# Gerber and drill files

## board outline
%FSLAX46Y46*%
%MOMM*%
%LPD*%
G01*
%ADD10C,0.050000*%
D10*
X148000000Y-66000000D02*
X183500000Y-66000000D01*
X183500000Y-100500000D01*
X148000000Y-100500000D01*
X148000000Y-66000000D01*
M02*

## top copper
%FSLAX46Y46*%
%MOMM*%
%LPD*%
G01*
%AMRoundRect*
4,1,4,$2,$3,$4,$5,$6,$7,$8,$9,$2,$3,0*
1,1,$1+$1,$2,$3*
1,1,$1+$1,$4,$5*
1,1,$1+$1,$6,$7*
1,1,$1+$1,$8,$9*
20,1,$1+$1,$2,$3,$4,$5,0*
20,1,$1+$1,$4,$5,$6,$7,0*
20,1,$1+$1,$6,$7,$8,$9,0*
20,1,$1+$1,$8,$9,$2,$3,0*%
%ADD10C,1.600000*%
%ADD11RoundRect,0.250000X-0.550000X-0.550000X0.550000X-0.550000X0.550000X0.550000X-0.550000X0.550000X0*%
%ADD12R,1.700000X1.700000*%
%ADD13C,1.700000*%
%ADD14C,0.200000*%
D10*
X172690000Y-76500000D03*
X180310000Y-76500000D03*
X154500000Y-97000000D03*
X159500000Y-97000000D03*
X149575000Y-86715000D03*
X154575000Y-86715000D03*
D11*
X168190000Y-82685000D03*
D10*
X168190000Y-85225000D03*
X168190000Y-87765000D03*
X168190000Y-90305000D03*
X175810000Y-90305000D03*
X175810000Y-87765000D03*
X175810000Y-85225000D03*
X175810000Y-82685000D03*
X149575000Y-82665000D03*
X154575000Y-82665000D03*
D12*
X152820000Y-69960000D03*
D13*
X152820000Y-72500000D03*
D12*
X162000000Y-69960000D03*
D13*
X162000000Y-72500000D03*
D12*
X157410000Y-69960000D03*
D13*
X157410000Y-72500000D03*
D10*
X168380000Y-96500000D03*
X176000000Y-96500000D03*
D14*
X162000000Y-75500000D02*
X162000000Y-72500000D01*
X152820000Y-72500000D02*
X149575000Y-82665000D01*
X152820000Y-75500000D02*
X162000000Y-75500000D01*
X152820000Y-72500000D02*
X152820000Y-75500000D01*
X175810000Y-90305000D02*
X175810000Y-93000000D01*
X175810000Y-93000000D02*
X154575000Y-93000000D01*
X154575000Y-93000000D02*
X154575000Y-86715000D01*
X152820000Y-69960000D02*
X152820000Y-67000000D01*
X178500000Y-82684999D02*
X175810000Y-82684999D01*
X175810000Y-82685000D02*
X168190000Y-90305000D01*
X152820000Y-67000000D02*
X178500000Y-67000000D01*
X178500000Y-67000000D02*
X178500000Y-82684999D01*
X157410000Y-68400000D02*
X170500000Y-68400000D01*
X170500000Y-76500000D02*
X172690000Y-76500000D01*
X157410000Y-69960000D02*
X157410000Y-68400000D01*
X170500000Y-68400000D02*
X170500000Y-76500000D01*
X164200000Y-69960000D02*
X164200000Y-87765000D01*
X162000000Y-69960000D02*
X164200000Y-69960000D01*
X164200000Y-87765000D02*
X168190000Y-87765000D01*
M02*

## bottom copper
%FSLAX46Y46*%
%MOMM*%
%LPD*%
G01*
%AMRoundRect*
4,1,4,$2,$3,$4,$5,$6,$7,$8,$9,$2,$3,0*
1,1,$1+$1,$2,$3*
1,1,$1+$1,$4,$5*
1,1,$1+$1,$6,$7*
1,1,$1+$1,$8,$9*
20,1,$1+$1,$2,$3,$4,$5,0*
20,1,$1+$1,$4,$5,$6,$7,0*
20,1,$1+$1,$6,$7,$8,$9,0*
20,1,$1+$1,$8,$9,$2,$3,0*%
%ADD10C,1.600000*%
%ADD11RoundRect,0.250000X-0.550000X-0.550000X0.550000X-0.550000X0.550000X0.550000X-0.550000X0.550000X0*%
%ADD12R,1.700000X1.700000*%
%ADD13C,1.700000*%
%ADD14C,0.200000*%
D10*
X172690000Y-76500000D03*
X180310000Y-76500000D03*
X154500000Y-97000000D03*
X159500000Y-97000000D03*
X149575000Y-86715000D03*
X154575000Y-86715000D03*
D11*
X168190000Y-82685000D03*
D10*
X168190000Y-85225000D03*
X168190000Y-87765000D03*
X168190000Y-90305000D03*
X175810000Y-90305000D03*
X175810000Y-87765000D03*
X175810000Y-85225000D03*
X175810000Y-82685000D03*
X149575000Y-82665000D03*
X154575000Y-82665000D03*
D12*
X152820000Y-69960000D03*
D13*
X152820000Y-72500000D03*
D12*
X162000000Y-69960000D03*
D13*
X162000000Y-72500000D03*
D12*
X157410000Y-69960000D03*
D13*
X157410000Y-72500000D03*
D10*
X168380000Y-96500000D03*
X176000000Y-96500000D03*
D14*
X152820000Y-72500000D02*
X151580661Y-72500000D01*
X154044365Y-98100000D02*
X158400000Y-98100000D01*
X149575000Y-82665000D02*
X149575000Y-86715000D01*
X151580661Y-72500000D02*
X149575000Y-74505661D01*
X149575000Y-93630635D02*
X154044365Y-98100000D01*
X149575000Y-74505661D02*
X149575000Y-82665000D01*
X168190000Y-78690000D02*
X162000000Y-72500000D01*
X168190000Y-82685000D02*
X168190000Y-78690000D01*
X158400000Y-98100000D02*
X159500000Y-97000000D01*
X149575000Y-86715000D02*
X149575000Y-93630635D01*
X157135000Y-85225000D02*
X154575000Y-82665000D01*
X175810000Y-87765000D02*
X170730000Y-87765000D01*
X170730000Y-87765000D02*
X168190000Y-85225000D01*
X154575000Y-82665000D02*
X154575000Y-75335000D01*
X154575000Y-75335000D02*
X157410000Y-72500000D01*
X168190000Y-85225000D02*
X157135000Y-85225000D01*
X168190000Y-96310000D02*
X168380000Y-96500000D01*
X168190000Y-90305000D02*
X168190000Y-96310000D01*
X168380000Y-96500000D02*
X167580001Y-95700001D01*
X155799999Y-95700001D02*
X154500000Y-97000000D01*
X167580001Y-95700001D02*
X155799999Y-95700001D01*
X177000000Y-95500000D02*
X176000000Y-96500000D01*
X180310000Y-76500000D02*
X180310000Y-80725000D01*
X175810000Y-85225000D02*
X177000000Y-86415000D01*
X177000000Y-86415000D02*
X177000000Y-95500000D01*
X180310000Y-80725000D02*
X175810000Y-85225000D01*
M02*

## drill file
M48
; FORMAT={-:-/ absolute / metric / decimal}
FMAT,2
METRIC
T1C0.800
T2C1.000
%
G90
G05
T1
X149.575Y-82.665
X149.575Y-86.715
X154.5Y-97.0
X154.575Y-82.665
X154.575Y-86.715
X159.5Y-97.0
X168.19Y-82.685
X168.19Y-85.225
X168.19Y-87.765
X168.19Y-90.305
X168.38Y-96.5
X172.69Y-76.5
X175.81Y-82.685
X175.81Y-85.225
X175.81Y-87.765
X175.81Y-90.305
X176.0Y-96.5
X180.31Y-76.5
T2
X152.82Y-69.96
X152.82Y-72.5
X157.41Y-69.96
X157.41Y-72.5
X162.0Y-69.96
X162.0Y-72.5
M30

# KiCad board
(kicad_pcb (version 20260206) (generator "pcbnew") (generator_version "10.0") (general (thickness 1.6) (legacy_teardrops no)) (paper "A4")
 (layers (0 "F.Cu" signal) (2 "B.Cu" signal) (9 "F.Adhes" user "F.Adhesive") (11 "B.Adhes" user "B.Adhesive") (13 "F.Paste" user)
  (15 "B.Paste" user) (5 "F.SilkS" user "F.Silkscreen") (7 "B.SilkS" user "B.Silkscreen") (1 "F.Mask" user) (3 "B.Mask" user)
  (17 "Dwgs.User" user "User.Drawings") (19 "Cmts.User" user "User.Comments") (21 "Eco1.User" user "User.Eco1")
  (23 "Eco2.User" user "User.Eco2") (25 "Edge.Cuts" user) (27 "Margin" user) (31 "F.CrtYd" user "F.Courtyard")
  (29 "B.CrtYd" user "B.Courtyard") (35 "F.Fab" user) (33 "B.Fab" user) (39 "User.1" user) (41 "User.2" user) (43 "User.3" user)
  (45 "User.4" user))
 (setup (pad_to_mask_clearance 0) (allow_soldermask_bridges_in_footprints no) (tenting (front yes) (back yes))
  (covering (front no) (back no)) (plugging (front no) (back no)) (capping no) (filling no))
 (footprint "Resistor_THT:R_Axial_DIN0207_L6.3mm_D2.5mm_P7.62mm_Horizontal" (layer "F.Cu") (at 172.69 76.5)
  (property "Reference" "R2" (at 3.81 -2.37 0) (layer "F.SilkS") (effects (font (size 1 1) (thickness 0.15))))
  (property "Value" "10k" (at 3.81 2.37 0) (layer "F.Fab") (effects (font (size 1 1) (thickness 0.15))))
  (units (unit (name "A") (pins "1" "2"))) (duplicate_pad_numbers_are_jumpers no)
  (pad "1" thru_hole circle (at 0 0) (size 1.6 1.6) (drill 0.8) (layers "*.Cu" "*.Mask") (remove_unused_layers no) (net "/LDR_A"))
  (pad "2" thru_hole circle (at 7.62 0) (size 1.6 1.6) (drill 0.8) (layers "*.Cu" "*.Mask") (remove_unused_layers no) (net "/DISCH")))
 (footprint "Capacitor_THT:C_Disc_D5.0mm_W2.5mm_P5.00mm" (layer "F.Cu") (at 154.5 97)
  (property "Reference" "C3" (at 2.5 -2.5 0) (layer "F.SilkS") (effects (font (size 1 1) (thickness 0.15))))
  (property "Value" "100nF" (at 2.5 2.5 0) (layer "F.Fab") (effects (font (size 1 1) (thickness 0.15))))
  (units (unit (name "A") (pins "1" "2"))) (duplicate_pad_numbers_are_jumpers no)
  (pad "1" thru_hole circle (at 0 0) (size 1.6 1.6) (drill 0.8) (layers "*.Cu" "*.Mask") (remove_unused_layers no) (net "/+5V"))
  (pad "2" thru_hole circle (at 5 0) (size 1.6 1.6) (drill 0.8) (layers "*.Cu" "*.Mask") (remove_unused_layers no) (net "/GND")))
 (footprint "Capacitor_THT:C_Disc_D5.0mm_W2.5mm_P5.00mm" (layer "F.Cu") (at 149.575 86.715)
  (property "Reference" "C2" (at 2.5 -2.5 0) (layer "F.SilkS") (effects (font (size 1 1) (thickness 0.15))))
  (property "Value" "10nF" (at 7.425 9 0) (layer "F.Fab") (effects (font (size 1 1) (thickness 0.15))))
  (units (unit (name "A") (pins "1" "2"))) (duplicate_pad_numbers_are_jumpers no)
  (pad "1" thru_hole circle (at 0 0) (size 1.6 1.6) (drill 0.8) (layers "*.Cu" "*.Mask") (remove_unused_layers no) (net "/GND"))
  (pad "2" thru_hole circle (at 5 0) (size 1.6 1.6) (drill 0.8) (layers "*.Cu" "*.Mask") (remove_unused_layers no) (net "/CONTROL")))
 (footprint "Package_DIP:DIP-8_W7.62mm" (layer "F.Cu") (at 168.19 82.685)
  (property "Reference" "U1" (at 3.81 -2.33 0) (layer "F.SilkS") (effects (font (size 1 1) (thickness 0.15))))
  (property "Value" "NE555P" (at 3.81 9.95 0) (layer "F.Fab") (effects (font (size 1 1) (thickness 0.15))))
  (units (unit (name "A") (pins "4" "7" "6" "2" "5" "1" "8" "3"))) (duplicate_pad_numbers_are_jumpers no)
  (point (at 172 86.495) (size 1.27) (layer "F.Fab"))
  (pad "1" thru_hole roundrect (at 0 0) (size 1.6 1.6) (drill 0.8) (layers "*.Cu" "*.Mask") (remove_unused_layers no)
   (roundrect_rratio 0.15625) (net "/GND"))
  (pad "2" thru_hole circle (at 0 2.54) (size 1.6 1.6) (drill 0.8) (layers "*.Cu" "*.Mask") (remove_unused_layers no) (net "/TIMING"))
  (pad "3" thru_hole circle (at 0 5.08) (size 1.6 1.6) (drill 0.8) (layers "*.Cu" "*.Mask") (remove_unused_layers no) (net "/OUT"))
  (pad "4" thru_hole circle (at 0 7.62) (size 1.6 1.6) (drill 0.8) (layers "*.Cu" "*.Mask") (remove_unused_layers no) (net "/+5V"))
  (pad "5" thru_hole circle (at 7.62 7.62) (size 1.6 1.6) (drill 0.8) (layers "*.Cu" "*.Mask") (remove_unused_layers no) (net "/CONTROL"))
  (pad "6" thru_hole circle (at 7.62 5.08) (size 1.6 1.6) (drill 0.8) (layers "*.Cu" "*.Mask") (remove_unused_layers no) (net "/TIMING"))
  (pad "7" thru_hole circle (at 7.62 2.54) (size 1.6 1.6) (drill 0.8) (layers "*.Cu" "*.Mask") (remove_unused_layers no) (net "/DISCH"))
  (pad "8" thru_hole circle (at 7.62 0) (size 1.6 1.6) (drill 0.8) (layers "*.Cu" "*.Mask") (remove_unused_layers no) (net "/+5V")))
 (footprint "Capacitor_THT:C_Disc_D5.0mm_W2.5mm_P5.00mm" (layer "F.Cu") (at 149.575 82.665)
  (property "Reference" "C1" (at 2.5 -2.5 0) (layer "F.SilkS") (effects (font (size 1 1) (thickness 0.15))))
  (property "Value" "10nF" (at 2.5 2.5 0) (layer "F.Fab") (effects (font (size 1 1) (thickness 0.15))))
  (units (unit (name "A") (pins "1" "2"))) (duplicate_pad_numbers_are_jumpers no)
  (pad "1" thru_hole circle (at 0 0) (size 1.6 1.6) (drill 0.8) (layers "*.Cu" "*.Mask") (remove_unused_layers no) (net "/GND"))
  (pad "2" thru_hole circle (at 5 0) (size 1.6 1.6) (drill 0.8) (layers "*.Cu" "*.Mask") (remove_unused_layers no) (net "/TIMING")))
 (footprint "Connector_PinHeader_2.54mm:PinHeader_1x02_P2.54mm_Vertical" (layer "F.Cu") (at 152.82 69.96)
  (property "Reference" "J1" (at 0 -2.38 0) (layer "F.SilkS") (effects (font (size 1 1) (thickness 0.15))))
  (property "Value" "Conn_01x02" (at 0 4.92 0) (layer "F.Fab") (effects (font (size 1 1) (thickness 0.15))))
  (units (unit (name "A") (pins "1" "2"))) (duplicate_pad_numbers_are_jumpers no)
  (pad "1" thru_hole rect (at 0 0) (size 1.7 1.7) (drill 1) (layers "*.Cu" "*.Mask") (remove_unused_layers no) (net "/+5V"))
  (pad "2" thru_hole circle (at 0 2.54) (size 1.7 1.7) (drill 1) (layers "*.Cu" "*.Mask") (remove_unused_layers no) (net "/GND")))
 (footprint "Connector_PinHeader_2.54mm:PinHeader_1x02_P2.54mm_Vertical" (layer "F.Cu") (at 162 69.96)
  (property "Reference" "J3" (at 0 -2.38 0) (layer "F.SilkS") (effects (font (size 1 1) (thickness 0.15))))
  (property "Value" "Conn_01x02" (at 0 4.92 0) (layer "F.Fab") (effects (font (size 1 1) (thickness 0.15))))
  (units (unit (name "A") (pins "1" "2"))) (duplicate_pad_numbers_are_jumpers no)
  (pad "1" thru_hole rect (at 0 0) (size 1.7 1.7) (drill 1) (layers "*.Cu" "*.Mask") (remove_unused_layers no) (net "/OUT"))
  (pad "2" thru_hole circle (at 0 2.54) (size 1.7 1.7) (drill 1) (layers "*.Cu" "*.Mask") (remove_unused_layers no) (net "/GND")))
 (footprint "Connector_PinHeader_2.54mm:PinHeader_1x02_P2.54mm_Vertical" (layer "F.Cu") (at 157.41 69.96)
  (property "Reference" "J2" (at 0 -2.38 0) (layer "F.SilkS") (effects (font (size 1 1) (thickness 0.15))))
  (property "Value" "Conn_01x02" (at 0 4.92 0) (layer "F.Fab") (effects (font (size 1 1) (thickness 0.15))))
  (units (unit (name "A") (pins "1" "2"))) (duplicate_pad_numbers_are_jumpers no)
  (pad "1" thru_hole rect (at 0 0) (size 1.7 1.7) (drill 1) (layers "*.Cu" "*.Mask") (remove_unused_layers no) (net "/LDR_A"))
  (pad "2" thru_hole circle (at 0 2.54) (size 1.7 1.7) (drill 1) (layers "*.Cu" "*.Mask") (remove_unused_layers no) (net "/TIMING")))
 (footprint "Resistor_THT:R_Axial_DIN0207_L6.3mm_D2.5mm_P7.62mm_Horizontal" (layer "F.Cu") (at 168.38 96.5)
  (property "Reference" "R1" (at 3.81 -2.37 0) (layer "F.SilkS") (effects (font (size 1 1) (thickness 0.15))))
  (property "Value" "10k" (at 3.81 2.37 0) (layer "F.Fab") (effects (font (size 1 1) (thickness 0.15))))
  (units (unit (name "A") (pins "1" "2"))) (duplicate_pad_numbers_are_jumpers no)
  (pad "1" thru_hole circle (at 0 0) (size 1.6 1.6) (drill 0.8) (layers "*.Cu" "*.Mask") (remove_unused_layers no) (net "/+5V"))
  (pad "2" thru_hole circle (at 7.62 0) (size 1.6 1.6) (drill 0.8) (layers "*.Cu" "*.Mask") (remove_unused_layers no) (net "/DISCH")))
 (gr_rect (start 148 66) (end 183.5 100.5) (stroke (width 0.05) (type default)) (fill no) (layer "Edge.Cuts"))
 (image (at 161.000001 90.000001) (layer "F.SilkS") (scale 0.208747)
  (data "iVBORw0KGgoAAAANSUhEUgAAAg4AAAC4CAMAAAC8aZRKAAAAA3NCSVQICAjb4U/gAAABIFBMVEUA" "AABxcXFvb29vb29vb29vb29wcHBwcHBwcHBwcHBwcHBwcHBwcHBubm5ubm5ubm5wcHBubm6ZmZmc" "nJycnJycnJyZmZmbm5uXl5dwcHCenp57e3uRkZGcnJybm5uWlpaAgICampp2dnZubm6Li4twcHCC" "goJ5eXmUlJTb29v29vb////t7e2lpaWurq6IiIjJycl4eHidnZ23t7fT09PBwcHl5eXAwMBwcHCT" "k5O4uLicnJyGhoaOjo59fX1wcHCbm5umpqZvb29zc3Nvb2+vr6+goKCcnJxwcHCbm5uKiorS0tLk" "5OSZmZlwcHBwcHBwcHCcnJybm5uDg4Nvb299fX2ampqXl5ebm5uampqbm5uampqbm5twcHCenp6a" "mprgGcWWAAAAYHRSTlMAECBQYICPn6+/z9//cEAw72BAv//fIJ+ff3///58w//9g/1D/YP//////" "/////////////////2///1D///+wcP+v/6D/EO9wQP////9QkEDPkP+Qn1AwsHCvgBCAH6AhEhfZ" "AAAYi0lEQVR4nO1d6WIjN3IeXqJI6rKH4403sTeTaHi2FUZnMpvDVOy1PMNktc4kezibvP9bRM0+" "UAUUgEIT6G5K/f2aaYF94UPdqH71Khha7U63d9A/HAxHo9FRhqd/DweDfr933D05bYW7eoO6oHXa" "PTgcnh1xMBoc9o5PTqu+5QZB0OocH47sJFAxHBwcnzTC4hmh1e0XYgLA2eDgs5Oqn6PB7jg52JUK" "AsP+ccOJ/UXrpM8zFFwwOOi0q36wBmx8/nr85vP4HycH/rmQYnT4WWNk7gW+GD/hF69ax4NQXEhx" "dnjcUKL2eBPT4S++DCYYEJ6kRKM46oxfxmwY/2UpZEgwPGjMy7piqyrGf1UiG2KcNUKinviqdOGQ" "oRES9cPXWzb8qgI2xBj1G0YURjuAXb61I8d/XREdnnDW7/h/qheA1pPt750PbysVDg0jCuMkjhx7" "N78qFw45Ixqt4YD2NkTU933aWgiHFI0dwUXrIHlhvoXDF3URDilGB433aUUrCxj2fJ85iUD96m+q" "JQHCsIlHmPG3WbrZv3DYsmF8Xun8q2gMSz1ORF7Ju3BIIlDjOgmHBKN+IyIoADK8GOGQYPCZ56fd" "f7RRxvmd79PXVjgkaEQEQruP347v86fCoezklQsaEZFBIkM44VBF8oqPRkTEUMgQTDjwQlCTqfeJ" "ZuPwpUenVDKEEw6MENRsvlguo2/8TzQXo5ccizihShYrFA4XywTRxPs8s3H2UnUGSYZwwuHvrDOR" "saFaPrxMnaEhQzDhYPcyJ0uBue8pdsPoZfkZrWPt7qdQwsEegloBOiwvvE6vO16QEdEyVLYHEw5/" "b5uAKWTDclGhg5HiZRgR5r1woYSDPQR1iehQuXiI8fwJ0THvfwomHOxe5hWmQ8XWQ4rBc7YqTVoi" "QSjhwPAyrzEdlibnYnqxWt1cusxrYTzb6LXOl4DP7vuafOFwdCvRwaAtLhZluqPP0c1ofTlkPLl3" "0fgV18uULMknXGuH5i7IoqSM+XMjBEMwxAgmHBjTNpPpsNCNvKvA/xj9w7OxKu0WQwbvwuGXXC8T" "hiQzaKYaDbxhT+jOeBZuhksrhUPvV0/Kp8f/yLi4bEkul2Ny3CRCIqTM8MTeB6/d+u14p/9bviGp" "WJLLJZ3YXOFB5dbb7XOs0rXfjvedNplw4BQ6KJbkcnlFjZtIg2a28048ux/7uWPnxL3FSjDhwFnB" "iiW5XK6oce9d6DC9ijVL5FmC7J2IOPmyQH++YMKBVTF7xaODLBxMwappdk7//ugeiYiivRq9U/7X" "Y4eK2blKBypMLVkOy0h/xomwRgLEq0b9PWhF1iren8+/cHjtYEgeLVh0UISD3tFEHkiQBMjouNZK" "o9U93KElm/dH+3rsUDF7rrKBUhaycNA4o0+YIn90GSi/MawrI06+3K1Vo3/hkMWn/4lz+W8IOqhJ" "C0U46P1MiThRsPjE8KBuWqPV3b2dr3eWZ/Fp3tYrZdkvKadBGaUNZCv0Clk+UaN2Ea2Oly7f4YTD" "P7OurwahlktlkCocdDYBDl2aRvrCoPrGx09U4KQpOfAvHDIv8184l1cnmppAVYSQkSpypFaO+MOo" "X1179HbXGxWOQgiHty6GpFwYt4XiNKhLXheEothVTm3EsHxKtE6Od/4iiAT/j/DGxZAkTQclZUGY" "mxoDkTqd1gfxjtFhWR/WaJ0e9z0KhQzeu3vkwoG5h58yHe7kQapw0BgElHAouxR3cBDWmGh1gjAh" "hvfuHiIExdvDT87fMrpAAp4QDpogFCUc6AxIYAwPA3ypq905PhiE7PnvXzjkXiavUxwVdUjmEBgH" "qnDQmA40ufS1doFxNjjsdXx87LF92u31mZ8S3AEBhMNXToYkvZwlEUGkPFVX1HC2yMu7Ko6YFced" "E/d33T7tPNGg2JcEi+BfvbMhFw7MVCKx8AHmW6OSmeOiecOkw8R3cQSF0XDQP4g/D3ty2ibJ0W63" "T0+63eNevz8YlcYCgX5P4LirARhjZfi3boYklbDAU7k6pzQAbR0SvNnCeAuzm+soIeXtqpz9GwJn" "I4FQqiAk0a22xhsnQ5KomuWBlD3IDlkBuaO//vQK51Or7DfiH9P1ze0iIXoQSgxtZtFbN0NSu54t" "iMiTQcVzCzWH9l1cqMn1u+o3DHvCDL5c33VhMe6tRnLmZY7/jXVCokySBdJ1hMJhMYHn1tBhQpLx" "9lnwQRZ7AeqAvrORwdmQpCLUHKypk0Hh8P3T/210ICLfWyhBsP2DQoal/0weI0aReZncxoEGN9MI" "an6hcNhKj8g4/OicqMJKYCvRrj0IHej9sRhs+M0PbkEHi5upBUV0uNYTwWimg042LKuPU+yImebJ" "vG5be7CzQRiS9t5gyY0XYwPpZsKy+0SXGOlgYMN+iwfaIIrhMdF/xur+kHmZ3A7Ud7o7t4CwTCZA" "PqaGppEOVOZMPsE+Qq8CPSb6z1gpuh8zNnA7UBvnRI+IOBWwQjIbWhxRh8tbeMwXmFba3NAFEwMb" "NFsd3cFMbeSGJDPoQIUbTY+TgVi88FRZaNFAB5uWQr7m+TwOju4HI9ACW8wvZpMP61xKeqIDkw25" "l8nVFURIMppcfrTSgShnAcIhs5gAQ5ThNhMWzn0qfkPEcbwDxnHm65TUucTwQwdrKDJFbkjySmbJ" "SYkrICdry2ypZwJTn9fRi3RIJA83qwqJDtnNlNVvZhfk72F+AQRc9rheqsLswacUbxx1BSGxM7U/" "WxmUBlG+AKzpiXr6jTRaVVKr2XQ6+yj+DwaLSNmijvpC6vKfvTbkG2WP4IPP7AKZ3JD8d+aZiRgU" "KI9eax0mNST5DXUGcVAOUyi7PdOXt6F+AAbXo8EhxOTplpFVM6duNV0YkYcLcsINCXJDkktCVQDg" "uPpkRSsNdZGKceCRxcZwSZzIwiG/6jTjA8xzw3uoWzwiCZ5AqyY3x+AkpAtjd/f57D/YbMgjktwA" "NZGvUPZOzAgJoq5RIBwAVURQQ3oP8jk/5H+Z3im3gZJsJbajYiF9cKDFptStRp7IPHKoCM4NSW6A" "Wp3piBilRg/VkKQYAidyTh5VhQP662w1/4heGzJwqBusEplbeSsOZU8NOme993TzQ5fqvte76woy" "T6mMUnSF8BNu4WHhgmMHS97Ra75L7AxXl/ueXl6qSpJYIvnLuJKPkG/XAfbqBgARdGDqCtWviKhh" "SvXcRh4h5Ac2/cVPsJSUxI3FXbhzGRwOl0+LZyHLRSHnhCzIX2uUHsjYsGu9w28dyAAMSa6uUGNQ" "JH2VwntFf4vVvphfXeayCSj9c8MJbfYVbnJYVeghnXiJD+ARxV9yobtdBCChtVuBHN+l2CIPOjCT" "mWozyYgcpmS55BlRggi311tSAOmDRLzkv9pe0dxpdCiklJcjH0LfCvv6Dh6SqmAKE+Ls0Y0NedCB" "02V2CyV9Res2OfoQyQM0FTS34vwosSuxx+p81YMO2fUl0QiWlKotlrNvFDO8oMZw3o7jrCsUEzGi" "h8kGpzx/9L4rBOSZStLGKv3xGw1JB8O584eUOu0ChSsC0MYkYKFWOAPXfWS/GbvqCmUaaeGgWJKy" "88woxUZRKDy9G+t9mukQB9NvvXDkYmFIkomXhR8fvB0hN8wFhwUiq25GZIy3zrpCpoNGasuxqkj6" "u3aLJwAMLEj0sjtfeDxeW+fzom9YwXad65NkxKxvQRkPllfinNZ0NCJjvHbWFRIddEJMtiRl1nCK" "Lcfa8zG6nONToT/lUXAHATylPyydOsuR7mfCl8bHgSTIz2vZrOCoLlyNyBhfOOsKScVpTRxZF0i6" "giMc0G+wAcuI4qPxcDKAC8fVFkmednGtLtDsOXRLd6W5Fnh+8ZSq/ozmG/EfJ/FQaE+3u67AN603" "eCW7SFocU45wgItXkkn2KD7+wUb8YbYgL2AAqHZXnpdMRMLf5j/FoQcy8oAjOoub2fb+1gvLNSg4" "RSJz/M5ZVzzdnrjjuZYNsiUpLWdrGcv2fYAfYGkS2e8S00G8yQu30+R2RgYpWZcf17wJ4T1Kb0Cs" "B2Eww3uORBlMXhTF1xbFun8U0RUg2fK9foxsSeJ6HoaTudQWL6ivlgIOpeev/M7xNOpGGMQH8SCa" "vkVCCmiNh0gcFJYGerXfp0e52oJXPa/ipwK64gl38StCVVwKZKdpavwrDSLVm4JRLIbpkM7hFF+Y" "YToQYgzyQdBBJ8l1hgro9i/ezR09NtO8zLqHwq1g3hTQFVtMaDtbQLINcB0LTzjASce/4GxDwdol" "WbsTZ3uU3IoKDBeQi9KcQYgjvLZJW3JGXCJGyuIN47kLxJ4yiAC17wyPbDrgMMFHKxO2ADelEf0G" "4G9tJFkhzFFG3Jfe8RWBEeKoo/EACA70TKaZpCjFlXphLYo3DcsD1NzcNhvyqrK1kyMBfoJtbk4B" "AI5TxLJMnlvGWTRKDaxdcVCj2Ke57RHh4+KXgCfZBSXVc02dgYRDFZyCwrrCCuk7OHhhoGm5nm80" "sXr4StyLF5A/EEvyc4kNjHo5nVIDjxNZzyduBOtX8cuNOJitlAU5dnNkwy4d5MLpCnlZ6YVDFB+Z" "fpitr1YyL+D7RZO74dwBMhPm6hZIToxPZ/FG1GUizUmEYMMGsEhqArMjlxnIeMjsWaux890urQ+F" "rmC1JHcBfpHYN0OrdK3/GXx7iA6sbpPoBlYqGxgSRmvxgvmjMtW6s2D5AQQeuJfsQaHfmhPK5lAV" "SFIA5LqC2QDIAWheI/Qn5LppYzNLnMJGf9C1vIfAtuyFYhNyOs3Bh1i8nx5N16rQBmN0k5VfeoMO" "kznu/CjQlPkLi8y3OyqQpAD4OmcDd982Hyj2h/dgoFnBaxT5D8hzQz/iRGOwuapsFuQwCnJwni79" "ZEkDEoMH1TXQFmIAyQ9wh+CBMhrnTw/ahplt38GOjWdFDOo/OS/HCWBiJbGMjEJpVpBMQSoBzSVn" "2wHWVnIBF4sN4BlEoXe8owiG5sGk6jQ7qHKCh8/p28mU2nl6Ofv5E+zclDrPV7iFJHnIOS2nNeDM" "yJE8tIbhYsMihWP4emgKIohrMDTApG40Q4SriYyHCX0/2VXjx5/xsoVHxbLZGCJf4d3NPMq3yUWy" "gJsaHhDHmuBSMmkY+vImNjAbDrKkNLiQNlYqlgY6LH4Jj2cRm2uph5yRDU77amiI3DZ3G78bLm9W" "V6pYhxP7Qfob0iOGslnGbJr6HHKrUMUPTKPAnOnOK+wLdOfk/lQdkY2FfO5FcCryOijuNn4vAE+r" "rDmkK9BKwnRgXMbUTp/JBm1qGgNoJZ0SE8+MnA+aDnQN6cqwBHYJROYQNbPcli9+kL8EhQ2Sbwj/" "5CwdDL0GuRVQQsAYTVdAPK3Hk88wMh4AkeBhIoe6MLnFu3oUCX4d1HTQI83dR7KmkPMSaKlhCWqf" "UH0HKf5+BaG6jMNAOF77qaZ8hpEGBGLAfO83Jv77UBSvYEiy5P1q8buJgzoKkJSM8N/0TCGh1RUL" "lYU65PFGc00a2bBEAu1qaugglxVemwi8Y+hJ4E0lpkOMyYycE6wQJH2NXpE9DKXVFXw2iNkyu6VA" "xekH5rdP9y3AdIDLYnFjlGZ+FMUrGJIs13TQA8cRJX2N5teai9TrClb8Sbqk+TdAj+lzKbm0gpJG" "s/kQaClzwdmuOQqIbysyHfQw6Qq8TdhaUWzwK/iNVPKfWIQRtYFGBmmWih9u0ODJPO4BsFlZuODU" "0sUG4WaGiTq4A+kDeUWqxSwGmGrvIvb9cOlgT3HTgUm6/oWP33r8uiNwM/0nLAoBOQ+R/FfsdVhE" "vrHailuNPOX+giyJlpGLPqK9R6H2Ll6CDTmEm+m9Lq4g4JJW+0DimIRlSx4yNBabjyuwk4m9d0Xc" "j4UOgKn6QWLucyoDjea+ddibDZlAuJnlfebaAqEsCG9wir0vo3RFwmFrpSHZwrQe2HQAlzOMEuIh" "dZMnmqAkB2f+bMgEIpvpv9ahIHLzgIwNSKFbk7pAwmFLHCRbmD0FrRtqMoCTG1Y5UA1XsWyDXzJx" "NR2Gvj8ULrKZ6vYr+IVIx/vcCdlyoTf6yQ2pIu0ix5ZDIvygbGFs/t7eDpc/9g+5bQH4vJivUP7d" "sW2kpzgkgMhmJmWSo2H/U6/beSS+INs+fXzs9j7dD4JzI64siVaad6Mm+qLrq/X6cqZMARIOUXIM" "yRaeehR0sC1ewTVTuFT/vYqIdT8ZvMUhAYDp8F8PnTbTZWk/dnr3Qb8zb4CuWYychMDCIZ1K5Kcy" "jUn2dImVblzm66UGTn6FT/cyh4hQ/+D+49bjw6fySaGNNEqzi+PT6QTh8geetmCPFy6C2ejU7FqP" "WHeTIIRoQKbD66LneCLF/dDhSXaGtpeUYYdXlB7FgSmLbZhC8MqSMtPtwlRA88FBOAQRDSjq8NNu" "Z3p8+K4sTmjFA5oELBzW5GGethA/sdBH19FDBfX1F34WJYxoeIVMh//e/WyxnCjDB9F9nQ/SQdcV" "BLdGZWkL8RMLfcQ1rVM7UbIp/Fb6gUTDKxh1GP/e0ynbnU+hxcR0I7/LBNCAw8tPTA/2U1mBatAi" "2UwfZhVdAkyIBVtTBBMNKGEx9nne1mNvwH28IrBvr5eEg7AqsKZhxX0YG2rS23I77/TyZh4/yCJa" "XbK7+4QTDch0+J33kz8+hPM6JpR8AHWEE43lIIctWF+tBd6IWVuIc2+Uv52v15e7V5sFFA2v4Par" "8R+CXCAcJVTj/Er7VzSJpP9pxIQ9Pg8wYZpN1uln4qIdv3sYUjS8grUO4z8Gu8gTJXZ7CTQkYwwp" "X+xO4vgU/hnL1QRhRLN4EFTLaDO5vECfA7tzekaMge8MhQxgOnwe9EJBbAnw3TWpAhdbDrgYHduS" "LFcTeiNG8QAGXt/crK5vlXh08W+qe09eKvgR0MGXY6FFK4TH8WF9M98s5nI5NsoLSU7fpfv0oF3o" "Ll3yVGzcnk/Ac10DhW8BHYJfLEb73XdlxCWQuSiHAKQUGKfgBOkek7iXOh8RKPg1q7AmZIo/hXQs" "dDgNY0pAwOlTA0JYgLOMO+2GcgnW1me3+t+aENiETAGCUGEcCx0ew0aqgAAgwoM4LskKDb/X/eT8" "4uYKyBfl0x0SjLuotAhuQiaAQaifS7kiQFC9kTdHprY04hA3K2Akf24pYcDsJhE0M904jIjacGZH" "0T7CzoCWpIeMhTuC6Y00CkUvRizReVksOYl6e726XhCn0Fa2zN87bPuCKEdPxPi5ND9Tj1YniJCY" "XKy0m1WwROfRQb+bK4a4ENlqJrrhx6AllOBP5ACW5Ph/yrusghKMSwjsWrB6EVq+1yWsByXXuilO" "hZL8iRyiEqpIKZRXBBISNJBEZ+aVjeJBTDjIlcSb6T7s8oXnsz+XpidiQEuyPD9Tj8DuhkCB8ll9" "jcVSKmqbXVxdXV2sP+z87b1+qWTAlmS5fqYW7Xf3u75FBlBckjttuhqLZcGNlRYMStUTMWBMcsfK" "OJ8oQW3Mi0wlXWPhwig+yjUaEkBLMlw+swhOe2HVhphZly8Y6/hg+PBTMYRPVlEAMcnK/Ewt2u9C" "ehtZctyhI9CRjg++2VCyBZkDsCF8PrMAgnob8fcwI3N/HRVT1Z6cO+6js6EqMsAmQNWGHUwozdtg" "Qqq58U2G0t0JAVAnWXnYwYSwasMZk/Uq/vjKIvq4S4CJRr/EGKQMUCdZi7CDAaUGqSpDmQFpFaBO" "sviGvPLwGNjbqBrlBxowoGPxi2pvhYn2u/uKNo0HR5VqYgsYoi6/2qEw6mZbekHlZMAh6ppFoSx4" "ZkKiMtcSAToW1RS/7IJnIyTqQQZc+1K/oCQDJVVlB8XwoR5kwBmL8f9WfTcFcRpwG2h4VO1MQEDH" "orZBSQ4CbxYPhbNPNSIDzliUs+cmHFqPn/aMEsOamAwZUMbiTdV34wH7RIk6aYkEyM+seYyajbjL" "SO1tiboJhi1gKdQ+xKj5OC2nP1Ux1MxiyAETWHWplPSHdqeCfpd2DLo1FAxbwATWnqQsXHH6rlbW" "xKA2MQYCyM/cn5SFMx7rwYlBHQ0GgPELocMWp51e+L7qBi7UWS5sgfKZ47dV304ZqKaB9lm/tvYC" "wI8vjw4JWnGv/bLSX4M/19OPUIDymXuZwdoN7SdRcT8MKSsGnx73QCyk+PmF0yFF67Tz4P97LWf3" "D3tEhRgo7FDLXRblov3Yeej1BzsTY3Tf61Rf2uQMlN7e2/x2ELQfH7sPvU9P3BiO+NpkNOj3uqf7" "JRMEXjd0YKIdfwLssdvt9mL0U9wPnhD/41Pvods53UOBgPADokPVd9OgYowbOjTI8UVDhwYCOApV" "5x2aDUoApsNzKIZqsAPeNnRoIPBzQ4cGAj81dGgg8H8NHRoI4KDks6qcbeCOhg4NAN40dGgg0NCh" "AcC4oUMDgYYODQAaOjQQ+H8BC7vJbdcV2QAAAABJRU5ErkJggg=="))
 (segment (start 162 75.5) (end 162 72.5) (width 0.2) (layer "F.Cu") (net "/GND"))
 (segment (start 152.82 72.5) (end 149.575 82.665) (width 0.2) (layer "F.Cu") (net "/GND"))
 (segment (start 152.82 75.5) (end 162 75.5) (width 0.2) (layer "F.Cu") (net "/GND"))
 (segment (start 152.82 72.5) (end 152.82 75.5) (width 0.2) (layer "F.Cu") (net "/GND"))
 (segment (start 152.82 72.5) (end 151.580661 72.5) (width 0.2) (layer "B.Cu") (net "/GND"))
 (segment (start 154.044365 98.1) (end 158.4 98.1) (width 0.2) (layer "B.Cu") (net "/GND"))
 (segment (start 149.575 82.665) (end 149.575 86.715) (width 0.2) (layer "B.Cu") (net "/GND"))
 (segment (start 151.580661 72.5) (end 149.575 74.505661) (width 0.2) (layer "B.Cu") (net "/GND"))
 (segment (start 149.575 93.630635) (end 154.044365 98.1) (width 0.2) (layer "B.Cu") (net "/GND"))
 (segment (start 149.575 74.505661) (end 149.575 82.665) (width 0.2) (layer "B.Cu") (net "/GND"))
 (segment (start 168.19 78.69) (end 162 72.5) (width 0.2) (layer "B.Cu") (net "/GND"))
 (segment (start 168.19 82.685) (end 168.19 78.69) (width 0.2) (layer "B.Cu") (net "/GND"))
 (segment (start 158.4 98.1) (end 159.5 97) (width 0.2) (layer "B.Cu") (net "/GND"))
 (segment (start 149.575 86.715) (end 149.575 93.630635) (width 0.2) (layer "B.Cu") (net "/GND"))
 (segment (start 157.135 85.225) (end 154.575 82.665) (width 0.2) (layer "B.Cu") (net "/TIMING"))
 (segment (start 175.81 87.765) (end 170.73 87.765) (width 0.2) (layer "B.Cu") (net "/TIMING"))
 (segment (start 170.73 87.765) (end 168.19 85.225) (width 0.2) (layer "B.Cu") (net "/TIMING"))
 (segment (start 154.575 82.665) (end 154.575 75.335) (width 0.2) (layer "B.Cu") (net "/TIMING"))
 (segment (start 154.575 75.335) (end 157.41 72.5) (width 0.2) (layer "B.Cu") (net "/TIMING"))
 (segment (start 168.19 85.225) (end 157.135 85.225) (width 0.2) (layer "B.Cu") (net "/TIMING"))
 (segment (start 175.81 90.305) (end 175.81 93) (width 0.2) (layer "F.Cu") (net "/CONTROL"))
 (segment (start 175.81 93) (end 154.575 93) (width 0.2) (layer "F.Cu") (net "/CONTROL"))
 (segment (start 154.575 93) (end 154.575 86.715) (width 0.2) (layer "F.Cu") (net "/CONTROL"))
 (segment (start 152.82 69.96) (end 152.82 67) (width 0.2) (layer "F.Cu") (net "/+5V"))
 (segment (start 178.5 82.684999) (end 175.81 82.684999) (width 0.2) (layer "F.Cu") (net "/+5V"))
 (segment (start 175.81 82.685) (end 168.19 90.305) (width 0.2) (layer "F.Cu") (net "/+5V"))
 (segment (start 152.82 67) (end 178.5 67) (width 0.2) (layer "F.Cu") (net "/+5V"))
 (segment (start 178.5 67) (end 178.5 82.684999) (width 0.2) (layer "F.Cu") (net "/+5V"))
 (segment (start 168.19 96.31) (end 168.38 96.5) (width 0.2) (layer "B.Cu") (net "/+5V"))
 (segment (start 168.19 90.305) (end 168.19 96.31) (width 0.2) (layer "B.Cu") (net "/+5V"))
 (segment (start 168.38 96.5) (end 167.580001 95.700001) (width 0.2) (layer "B.Cu") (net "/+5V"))
 (segment (start 155.799999 95.700001) (end 154.5 97) (width 0.2) (layer "B.Cu") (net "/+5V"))
 (segment (start 167.580001 95.700001) (end 155.799999 95.700001) (width 0.2) (layer "B.Cu") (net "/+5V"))
 (segment (start 157.41 68.4) (end 170.5 68.4) (width 0.2) (layer "F.Cu") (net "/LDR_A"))
 (segment (start 170.5 76.5) (end 172.69 76.5) (width 0.2) (layer "F.Cu") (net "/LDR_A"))
 (segment (start 157.41 69.96) (end 157.41 68.4) (width 0.2) (layer "F.Cu") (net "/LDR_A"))
 (segment (start 170.5 68.4) (end 170.5 76.5) (width 0.2) (layer "F.Cu") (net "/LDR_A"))
 (segment (start 164.2 69.96) (end 164.2 87.765) (width 0.2) (layer "F.Cu") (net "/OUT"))
 (segment (start 162 69.96) (end 164.2 69.96) (width 0.2) (layer "F.Cu") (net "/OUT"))
 (segment (start 164.2 87.765) (end 168.19 87.765) (width 0.2) (layer "F.Cu") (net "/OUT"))
 (segment (start 177 95.5) (end 176 96.5) (width 0.2) (layer "B.Cu") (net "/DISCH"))
 (segment (start 180.31 76.5) (end 180.31 80.725) (width 0.2) (layer "B.Cu") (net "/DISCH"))
 (segment (start 175.81 85.225) (end 177 86.415) (width 0.2) (layer "B.Cu") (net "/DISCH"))
 (segment (start 177 86.415) (end 177 95.5) (width 0.2) (layer "B.Cu") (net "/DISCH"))
 (segment (start 180.31 80.725) (end 175.81 85.225) (width 0.2) (layer "B.Cu") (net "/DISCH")))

